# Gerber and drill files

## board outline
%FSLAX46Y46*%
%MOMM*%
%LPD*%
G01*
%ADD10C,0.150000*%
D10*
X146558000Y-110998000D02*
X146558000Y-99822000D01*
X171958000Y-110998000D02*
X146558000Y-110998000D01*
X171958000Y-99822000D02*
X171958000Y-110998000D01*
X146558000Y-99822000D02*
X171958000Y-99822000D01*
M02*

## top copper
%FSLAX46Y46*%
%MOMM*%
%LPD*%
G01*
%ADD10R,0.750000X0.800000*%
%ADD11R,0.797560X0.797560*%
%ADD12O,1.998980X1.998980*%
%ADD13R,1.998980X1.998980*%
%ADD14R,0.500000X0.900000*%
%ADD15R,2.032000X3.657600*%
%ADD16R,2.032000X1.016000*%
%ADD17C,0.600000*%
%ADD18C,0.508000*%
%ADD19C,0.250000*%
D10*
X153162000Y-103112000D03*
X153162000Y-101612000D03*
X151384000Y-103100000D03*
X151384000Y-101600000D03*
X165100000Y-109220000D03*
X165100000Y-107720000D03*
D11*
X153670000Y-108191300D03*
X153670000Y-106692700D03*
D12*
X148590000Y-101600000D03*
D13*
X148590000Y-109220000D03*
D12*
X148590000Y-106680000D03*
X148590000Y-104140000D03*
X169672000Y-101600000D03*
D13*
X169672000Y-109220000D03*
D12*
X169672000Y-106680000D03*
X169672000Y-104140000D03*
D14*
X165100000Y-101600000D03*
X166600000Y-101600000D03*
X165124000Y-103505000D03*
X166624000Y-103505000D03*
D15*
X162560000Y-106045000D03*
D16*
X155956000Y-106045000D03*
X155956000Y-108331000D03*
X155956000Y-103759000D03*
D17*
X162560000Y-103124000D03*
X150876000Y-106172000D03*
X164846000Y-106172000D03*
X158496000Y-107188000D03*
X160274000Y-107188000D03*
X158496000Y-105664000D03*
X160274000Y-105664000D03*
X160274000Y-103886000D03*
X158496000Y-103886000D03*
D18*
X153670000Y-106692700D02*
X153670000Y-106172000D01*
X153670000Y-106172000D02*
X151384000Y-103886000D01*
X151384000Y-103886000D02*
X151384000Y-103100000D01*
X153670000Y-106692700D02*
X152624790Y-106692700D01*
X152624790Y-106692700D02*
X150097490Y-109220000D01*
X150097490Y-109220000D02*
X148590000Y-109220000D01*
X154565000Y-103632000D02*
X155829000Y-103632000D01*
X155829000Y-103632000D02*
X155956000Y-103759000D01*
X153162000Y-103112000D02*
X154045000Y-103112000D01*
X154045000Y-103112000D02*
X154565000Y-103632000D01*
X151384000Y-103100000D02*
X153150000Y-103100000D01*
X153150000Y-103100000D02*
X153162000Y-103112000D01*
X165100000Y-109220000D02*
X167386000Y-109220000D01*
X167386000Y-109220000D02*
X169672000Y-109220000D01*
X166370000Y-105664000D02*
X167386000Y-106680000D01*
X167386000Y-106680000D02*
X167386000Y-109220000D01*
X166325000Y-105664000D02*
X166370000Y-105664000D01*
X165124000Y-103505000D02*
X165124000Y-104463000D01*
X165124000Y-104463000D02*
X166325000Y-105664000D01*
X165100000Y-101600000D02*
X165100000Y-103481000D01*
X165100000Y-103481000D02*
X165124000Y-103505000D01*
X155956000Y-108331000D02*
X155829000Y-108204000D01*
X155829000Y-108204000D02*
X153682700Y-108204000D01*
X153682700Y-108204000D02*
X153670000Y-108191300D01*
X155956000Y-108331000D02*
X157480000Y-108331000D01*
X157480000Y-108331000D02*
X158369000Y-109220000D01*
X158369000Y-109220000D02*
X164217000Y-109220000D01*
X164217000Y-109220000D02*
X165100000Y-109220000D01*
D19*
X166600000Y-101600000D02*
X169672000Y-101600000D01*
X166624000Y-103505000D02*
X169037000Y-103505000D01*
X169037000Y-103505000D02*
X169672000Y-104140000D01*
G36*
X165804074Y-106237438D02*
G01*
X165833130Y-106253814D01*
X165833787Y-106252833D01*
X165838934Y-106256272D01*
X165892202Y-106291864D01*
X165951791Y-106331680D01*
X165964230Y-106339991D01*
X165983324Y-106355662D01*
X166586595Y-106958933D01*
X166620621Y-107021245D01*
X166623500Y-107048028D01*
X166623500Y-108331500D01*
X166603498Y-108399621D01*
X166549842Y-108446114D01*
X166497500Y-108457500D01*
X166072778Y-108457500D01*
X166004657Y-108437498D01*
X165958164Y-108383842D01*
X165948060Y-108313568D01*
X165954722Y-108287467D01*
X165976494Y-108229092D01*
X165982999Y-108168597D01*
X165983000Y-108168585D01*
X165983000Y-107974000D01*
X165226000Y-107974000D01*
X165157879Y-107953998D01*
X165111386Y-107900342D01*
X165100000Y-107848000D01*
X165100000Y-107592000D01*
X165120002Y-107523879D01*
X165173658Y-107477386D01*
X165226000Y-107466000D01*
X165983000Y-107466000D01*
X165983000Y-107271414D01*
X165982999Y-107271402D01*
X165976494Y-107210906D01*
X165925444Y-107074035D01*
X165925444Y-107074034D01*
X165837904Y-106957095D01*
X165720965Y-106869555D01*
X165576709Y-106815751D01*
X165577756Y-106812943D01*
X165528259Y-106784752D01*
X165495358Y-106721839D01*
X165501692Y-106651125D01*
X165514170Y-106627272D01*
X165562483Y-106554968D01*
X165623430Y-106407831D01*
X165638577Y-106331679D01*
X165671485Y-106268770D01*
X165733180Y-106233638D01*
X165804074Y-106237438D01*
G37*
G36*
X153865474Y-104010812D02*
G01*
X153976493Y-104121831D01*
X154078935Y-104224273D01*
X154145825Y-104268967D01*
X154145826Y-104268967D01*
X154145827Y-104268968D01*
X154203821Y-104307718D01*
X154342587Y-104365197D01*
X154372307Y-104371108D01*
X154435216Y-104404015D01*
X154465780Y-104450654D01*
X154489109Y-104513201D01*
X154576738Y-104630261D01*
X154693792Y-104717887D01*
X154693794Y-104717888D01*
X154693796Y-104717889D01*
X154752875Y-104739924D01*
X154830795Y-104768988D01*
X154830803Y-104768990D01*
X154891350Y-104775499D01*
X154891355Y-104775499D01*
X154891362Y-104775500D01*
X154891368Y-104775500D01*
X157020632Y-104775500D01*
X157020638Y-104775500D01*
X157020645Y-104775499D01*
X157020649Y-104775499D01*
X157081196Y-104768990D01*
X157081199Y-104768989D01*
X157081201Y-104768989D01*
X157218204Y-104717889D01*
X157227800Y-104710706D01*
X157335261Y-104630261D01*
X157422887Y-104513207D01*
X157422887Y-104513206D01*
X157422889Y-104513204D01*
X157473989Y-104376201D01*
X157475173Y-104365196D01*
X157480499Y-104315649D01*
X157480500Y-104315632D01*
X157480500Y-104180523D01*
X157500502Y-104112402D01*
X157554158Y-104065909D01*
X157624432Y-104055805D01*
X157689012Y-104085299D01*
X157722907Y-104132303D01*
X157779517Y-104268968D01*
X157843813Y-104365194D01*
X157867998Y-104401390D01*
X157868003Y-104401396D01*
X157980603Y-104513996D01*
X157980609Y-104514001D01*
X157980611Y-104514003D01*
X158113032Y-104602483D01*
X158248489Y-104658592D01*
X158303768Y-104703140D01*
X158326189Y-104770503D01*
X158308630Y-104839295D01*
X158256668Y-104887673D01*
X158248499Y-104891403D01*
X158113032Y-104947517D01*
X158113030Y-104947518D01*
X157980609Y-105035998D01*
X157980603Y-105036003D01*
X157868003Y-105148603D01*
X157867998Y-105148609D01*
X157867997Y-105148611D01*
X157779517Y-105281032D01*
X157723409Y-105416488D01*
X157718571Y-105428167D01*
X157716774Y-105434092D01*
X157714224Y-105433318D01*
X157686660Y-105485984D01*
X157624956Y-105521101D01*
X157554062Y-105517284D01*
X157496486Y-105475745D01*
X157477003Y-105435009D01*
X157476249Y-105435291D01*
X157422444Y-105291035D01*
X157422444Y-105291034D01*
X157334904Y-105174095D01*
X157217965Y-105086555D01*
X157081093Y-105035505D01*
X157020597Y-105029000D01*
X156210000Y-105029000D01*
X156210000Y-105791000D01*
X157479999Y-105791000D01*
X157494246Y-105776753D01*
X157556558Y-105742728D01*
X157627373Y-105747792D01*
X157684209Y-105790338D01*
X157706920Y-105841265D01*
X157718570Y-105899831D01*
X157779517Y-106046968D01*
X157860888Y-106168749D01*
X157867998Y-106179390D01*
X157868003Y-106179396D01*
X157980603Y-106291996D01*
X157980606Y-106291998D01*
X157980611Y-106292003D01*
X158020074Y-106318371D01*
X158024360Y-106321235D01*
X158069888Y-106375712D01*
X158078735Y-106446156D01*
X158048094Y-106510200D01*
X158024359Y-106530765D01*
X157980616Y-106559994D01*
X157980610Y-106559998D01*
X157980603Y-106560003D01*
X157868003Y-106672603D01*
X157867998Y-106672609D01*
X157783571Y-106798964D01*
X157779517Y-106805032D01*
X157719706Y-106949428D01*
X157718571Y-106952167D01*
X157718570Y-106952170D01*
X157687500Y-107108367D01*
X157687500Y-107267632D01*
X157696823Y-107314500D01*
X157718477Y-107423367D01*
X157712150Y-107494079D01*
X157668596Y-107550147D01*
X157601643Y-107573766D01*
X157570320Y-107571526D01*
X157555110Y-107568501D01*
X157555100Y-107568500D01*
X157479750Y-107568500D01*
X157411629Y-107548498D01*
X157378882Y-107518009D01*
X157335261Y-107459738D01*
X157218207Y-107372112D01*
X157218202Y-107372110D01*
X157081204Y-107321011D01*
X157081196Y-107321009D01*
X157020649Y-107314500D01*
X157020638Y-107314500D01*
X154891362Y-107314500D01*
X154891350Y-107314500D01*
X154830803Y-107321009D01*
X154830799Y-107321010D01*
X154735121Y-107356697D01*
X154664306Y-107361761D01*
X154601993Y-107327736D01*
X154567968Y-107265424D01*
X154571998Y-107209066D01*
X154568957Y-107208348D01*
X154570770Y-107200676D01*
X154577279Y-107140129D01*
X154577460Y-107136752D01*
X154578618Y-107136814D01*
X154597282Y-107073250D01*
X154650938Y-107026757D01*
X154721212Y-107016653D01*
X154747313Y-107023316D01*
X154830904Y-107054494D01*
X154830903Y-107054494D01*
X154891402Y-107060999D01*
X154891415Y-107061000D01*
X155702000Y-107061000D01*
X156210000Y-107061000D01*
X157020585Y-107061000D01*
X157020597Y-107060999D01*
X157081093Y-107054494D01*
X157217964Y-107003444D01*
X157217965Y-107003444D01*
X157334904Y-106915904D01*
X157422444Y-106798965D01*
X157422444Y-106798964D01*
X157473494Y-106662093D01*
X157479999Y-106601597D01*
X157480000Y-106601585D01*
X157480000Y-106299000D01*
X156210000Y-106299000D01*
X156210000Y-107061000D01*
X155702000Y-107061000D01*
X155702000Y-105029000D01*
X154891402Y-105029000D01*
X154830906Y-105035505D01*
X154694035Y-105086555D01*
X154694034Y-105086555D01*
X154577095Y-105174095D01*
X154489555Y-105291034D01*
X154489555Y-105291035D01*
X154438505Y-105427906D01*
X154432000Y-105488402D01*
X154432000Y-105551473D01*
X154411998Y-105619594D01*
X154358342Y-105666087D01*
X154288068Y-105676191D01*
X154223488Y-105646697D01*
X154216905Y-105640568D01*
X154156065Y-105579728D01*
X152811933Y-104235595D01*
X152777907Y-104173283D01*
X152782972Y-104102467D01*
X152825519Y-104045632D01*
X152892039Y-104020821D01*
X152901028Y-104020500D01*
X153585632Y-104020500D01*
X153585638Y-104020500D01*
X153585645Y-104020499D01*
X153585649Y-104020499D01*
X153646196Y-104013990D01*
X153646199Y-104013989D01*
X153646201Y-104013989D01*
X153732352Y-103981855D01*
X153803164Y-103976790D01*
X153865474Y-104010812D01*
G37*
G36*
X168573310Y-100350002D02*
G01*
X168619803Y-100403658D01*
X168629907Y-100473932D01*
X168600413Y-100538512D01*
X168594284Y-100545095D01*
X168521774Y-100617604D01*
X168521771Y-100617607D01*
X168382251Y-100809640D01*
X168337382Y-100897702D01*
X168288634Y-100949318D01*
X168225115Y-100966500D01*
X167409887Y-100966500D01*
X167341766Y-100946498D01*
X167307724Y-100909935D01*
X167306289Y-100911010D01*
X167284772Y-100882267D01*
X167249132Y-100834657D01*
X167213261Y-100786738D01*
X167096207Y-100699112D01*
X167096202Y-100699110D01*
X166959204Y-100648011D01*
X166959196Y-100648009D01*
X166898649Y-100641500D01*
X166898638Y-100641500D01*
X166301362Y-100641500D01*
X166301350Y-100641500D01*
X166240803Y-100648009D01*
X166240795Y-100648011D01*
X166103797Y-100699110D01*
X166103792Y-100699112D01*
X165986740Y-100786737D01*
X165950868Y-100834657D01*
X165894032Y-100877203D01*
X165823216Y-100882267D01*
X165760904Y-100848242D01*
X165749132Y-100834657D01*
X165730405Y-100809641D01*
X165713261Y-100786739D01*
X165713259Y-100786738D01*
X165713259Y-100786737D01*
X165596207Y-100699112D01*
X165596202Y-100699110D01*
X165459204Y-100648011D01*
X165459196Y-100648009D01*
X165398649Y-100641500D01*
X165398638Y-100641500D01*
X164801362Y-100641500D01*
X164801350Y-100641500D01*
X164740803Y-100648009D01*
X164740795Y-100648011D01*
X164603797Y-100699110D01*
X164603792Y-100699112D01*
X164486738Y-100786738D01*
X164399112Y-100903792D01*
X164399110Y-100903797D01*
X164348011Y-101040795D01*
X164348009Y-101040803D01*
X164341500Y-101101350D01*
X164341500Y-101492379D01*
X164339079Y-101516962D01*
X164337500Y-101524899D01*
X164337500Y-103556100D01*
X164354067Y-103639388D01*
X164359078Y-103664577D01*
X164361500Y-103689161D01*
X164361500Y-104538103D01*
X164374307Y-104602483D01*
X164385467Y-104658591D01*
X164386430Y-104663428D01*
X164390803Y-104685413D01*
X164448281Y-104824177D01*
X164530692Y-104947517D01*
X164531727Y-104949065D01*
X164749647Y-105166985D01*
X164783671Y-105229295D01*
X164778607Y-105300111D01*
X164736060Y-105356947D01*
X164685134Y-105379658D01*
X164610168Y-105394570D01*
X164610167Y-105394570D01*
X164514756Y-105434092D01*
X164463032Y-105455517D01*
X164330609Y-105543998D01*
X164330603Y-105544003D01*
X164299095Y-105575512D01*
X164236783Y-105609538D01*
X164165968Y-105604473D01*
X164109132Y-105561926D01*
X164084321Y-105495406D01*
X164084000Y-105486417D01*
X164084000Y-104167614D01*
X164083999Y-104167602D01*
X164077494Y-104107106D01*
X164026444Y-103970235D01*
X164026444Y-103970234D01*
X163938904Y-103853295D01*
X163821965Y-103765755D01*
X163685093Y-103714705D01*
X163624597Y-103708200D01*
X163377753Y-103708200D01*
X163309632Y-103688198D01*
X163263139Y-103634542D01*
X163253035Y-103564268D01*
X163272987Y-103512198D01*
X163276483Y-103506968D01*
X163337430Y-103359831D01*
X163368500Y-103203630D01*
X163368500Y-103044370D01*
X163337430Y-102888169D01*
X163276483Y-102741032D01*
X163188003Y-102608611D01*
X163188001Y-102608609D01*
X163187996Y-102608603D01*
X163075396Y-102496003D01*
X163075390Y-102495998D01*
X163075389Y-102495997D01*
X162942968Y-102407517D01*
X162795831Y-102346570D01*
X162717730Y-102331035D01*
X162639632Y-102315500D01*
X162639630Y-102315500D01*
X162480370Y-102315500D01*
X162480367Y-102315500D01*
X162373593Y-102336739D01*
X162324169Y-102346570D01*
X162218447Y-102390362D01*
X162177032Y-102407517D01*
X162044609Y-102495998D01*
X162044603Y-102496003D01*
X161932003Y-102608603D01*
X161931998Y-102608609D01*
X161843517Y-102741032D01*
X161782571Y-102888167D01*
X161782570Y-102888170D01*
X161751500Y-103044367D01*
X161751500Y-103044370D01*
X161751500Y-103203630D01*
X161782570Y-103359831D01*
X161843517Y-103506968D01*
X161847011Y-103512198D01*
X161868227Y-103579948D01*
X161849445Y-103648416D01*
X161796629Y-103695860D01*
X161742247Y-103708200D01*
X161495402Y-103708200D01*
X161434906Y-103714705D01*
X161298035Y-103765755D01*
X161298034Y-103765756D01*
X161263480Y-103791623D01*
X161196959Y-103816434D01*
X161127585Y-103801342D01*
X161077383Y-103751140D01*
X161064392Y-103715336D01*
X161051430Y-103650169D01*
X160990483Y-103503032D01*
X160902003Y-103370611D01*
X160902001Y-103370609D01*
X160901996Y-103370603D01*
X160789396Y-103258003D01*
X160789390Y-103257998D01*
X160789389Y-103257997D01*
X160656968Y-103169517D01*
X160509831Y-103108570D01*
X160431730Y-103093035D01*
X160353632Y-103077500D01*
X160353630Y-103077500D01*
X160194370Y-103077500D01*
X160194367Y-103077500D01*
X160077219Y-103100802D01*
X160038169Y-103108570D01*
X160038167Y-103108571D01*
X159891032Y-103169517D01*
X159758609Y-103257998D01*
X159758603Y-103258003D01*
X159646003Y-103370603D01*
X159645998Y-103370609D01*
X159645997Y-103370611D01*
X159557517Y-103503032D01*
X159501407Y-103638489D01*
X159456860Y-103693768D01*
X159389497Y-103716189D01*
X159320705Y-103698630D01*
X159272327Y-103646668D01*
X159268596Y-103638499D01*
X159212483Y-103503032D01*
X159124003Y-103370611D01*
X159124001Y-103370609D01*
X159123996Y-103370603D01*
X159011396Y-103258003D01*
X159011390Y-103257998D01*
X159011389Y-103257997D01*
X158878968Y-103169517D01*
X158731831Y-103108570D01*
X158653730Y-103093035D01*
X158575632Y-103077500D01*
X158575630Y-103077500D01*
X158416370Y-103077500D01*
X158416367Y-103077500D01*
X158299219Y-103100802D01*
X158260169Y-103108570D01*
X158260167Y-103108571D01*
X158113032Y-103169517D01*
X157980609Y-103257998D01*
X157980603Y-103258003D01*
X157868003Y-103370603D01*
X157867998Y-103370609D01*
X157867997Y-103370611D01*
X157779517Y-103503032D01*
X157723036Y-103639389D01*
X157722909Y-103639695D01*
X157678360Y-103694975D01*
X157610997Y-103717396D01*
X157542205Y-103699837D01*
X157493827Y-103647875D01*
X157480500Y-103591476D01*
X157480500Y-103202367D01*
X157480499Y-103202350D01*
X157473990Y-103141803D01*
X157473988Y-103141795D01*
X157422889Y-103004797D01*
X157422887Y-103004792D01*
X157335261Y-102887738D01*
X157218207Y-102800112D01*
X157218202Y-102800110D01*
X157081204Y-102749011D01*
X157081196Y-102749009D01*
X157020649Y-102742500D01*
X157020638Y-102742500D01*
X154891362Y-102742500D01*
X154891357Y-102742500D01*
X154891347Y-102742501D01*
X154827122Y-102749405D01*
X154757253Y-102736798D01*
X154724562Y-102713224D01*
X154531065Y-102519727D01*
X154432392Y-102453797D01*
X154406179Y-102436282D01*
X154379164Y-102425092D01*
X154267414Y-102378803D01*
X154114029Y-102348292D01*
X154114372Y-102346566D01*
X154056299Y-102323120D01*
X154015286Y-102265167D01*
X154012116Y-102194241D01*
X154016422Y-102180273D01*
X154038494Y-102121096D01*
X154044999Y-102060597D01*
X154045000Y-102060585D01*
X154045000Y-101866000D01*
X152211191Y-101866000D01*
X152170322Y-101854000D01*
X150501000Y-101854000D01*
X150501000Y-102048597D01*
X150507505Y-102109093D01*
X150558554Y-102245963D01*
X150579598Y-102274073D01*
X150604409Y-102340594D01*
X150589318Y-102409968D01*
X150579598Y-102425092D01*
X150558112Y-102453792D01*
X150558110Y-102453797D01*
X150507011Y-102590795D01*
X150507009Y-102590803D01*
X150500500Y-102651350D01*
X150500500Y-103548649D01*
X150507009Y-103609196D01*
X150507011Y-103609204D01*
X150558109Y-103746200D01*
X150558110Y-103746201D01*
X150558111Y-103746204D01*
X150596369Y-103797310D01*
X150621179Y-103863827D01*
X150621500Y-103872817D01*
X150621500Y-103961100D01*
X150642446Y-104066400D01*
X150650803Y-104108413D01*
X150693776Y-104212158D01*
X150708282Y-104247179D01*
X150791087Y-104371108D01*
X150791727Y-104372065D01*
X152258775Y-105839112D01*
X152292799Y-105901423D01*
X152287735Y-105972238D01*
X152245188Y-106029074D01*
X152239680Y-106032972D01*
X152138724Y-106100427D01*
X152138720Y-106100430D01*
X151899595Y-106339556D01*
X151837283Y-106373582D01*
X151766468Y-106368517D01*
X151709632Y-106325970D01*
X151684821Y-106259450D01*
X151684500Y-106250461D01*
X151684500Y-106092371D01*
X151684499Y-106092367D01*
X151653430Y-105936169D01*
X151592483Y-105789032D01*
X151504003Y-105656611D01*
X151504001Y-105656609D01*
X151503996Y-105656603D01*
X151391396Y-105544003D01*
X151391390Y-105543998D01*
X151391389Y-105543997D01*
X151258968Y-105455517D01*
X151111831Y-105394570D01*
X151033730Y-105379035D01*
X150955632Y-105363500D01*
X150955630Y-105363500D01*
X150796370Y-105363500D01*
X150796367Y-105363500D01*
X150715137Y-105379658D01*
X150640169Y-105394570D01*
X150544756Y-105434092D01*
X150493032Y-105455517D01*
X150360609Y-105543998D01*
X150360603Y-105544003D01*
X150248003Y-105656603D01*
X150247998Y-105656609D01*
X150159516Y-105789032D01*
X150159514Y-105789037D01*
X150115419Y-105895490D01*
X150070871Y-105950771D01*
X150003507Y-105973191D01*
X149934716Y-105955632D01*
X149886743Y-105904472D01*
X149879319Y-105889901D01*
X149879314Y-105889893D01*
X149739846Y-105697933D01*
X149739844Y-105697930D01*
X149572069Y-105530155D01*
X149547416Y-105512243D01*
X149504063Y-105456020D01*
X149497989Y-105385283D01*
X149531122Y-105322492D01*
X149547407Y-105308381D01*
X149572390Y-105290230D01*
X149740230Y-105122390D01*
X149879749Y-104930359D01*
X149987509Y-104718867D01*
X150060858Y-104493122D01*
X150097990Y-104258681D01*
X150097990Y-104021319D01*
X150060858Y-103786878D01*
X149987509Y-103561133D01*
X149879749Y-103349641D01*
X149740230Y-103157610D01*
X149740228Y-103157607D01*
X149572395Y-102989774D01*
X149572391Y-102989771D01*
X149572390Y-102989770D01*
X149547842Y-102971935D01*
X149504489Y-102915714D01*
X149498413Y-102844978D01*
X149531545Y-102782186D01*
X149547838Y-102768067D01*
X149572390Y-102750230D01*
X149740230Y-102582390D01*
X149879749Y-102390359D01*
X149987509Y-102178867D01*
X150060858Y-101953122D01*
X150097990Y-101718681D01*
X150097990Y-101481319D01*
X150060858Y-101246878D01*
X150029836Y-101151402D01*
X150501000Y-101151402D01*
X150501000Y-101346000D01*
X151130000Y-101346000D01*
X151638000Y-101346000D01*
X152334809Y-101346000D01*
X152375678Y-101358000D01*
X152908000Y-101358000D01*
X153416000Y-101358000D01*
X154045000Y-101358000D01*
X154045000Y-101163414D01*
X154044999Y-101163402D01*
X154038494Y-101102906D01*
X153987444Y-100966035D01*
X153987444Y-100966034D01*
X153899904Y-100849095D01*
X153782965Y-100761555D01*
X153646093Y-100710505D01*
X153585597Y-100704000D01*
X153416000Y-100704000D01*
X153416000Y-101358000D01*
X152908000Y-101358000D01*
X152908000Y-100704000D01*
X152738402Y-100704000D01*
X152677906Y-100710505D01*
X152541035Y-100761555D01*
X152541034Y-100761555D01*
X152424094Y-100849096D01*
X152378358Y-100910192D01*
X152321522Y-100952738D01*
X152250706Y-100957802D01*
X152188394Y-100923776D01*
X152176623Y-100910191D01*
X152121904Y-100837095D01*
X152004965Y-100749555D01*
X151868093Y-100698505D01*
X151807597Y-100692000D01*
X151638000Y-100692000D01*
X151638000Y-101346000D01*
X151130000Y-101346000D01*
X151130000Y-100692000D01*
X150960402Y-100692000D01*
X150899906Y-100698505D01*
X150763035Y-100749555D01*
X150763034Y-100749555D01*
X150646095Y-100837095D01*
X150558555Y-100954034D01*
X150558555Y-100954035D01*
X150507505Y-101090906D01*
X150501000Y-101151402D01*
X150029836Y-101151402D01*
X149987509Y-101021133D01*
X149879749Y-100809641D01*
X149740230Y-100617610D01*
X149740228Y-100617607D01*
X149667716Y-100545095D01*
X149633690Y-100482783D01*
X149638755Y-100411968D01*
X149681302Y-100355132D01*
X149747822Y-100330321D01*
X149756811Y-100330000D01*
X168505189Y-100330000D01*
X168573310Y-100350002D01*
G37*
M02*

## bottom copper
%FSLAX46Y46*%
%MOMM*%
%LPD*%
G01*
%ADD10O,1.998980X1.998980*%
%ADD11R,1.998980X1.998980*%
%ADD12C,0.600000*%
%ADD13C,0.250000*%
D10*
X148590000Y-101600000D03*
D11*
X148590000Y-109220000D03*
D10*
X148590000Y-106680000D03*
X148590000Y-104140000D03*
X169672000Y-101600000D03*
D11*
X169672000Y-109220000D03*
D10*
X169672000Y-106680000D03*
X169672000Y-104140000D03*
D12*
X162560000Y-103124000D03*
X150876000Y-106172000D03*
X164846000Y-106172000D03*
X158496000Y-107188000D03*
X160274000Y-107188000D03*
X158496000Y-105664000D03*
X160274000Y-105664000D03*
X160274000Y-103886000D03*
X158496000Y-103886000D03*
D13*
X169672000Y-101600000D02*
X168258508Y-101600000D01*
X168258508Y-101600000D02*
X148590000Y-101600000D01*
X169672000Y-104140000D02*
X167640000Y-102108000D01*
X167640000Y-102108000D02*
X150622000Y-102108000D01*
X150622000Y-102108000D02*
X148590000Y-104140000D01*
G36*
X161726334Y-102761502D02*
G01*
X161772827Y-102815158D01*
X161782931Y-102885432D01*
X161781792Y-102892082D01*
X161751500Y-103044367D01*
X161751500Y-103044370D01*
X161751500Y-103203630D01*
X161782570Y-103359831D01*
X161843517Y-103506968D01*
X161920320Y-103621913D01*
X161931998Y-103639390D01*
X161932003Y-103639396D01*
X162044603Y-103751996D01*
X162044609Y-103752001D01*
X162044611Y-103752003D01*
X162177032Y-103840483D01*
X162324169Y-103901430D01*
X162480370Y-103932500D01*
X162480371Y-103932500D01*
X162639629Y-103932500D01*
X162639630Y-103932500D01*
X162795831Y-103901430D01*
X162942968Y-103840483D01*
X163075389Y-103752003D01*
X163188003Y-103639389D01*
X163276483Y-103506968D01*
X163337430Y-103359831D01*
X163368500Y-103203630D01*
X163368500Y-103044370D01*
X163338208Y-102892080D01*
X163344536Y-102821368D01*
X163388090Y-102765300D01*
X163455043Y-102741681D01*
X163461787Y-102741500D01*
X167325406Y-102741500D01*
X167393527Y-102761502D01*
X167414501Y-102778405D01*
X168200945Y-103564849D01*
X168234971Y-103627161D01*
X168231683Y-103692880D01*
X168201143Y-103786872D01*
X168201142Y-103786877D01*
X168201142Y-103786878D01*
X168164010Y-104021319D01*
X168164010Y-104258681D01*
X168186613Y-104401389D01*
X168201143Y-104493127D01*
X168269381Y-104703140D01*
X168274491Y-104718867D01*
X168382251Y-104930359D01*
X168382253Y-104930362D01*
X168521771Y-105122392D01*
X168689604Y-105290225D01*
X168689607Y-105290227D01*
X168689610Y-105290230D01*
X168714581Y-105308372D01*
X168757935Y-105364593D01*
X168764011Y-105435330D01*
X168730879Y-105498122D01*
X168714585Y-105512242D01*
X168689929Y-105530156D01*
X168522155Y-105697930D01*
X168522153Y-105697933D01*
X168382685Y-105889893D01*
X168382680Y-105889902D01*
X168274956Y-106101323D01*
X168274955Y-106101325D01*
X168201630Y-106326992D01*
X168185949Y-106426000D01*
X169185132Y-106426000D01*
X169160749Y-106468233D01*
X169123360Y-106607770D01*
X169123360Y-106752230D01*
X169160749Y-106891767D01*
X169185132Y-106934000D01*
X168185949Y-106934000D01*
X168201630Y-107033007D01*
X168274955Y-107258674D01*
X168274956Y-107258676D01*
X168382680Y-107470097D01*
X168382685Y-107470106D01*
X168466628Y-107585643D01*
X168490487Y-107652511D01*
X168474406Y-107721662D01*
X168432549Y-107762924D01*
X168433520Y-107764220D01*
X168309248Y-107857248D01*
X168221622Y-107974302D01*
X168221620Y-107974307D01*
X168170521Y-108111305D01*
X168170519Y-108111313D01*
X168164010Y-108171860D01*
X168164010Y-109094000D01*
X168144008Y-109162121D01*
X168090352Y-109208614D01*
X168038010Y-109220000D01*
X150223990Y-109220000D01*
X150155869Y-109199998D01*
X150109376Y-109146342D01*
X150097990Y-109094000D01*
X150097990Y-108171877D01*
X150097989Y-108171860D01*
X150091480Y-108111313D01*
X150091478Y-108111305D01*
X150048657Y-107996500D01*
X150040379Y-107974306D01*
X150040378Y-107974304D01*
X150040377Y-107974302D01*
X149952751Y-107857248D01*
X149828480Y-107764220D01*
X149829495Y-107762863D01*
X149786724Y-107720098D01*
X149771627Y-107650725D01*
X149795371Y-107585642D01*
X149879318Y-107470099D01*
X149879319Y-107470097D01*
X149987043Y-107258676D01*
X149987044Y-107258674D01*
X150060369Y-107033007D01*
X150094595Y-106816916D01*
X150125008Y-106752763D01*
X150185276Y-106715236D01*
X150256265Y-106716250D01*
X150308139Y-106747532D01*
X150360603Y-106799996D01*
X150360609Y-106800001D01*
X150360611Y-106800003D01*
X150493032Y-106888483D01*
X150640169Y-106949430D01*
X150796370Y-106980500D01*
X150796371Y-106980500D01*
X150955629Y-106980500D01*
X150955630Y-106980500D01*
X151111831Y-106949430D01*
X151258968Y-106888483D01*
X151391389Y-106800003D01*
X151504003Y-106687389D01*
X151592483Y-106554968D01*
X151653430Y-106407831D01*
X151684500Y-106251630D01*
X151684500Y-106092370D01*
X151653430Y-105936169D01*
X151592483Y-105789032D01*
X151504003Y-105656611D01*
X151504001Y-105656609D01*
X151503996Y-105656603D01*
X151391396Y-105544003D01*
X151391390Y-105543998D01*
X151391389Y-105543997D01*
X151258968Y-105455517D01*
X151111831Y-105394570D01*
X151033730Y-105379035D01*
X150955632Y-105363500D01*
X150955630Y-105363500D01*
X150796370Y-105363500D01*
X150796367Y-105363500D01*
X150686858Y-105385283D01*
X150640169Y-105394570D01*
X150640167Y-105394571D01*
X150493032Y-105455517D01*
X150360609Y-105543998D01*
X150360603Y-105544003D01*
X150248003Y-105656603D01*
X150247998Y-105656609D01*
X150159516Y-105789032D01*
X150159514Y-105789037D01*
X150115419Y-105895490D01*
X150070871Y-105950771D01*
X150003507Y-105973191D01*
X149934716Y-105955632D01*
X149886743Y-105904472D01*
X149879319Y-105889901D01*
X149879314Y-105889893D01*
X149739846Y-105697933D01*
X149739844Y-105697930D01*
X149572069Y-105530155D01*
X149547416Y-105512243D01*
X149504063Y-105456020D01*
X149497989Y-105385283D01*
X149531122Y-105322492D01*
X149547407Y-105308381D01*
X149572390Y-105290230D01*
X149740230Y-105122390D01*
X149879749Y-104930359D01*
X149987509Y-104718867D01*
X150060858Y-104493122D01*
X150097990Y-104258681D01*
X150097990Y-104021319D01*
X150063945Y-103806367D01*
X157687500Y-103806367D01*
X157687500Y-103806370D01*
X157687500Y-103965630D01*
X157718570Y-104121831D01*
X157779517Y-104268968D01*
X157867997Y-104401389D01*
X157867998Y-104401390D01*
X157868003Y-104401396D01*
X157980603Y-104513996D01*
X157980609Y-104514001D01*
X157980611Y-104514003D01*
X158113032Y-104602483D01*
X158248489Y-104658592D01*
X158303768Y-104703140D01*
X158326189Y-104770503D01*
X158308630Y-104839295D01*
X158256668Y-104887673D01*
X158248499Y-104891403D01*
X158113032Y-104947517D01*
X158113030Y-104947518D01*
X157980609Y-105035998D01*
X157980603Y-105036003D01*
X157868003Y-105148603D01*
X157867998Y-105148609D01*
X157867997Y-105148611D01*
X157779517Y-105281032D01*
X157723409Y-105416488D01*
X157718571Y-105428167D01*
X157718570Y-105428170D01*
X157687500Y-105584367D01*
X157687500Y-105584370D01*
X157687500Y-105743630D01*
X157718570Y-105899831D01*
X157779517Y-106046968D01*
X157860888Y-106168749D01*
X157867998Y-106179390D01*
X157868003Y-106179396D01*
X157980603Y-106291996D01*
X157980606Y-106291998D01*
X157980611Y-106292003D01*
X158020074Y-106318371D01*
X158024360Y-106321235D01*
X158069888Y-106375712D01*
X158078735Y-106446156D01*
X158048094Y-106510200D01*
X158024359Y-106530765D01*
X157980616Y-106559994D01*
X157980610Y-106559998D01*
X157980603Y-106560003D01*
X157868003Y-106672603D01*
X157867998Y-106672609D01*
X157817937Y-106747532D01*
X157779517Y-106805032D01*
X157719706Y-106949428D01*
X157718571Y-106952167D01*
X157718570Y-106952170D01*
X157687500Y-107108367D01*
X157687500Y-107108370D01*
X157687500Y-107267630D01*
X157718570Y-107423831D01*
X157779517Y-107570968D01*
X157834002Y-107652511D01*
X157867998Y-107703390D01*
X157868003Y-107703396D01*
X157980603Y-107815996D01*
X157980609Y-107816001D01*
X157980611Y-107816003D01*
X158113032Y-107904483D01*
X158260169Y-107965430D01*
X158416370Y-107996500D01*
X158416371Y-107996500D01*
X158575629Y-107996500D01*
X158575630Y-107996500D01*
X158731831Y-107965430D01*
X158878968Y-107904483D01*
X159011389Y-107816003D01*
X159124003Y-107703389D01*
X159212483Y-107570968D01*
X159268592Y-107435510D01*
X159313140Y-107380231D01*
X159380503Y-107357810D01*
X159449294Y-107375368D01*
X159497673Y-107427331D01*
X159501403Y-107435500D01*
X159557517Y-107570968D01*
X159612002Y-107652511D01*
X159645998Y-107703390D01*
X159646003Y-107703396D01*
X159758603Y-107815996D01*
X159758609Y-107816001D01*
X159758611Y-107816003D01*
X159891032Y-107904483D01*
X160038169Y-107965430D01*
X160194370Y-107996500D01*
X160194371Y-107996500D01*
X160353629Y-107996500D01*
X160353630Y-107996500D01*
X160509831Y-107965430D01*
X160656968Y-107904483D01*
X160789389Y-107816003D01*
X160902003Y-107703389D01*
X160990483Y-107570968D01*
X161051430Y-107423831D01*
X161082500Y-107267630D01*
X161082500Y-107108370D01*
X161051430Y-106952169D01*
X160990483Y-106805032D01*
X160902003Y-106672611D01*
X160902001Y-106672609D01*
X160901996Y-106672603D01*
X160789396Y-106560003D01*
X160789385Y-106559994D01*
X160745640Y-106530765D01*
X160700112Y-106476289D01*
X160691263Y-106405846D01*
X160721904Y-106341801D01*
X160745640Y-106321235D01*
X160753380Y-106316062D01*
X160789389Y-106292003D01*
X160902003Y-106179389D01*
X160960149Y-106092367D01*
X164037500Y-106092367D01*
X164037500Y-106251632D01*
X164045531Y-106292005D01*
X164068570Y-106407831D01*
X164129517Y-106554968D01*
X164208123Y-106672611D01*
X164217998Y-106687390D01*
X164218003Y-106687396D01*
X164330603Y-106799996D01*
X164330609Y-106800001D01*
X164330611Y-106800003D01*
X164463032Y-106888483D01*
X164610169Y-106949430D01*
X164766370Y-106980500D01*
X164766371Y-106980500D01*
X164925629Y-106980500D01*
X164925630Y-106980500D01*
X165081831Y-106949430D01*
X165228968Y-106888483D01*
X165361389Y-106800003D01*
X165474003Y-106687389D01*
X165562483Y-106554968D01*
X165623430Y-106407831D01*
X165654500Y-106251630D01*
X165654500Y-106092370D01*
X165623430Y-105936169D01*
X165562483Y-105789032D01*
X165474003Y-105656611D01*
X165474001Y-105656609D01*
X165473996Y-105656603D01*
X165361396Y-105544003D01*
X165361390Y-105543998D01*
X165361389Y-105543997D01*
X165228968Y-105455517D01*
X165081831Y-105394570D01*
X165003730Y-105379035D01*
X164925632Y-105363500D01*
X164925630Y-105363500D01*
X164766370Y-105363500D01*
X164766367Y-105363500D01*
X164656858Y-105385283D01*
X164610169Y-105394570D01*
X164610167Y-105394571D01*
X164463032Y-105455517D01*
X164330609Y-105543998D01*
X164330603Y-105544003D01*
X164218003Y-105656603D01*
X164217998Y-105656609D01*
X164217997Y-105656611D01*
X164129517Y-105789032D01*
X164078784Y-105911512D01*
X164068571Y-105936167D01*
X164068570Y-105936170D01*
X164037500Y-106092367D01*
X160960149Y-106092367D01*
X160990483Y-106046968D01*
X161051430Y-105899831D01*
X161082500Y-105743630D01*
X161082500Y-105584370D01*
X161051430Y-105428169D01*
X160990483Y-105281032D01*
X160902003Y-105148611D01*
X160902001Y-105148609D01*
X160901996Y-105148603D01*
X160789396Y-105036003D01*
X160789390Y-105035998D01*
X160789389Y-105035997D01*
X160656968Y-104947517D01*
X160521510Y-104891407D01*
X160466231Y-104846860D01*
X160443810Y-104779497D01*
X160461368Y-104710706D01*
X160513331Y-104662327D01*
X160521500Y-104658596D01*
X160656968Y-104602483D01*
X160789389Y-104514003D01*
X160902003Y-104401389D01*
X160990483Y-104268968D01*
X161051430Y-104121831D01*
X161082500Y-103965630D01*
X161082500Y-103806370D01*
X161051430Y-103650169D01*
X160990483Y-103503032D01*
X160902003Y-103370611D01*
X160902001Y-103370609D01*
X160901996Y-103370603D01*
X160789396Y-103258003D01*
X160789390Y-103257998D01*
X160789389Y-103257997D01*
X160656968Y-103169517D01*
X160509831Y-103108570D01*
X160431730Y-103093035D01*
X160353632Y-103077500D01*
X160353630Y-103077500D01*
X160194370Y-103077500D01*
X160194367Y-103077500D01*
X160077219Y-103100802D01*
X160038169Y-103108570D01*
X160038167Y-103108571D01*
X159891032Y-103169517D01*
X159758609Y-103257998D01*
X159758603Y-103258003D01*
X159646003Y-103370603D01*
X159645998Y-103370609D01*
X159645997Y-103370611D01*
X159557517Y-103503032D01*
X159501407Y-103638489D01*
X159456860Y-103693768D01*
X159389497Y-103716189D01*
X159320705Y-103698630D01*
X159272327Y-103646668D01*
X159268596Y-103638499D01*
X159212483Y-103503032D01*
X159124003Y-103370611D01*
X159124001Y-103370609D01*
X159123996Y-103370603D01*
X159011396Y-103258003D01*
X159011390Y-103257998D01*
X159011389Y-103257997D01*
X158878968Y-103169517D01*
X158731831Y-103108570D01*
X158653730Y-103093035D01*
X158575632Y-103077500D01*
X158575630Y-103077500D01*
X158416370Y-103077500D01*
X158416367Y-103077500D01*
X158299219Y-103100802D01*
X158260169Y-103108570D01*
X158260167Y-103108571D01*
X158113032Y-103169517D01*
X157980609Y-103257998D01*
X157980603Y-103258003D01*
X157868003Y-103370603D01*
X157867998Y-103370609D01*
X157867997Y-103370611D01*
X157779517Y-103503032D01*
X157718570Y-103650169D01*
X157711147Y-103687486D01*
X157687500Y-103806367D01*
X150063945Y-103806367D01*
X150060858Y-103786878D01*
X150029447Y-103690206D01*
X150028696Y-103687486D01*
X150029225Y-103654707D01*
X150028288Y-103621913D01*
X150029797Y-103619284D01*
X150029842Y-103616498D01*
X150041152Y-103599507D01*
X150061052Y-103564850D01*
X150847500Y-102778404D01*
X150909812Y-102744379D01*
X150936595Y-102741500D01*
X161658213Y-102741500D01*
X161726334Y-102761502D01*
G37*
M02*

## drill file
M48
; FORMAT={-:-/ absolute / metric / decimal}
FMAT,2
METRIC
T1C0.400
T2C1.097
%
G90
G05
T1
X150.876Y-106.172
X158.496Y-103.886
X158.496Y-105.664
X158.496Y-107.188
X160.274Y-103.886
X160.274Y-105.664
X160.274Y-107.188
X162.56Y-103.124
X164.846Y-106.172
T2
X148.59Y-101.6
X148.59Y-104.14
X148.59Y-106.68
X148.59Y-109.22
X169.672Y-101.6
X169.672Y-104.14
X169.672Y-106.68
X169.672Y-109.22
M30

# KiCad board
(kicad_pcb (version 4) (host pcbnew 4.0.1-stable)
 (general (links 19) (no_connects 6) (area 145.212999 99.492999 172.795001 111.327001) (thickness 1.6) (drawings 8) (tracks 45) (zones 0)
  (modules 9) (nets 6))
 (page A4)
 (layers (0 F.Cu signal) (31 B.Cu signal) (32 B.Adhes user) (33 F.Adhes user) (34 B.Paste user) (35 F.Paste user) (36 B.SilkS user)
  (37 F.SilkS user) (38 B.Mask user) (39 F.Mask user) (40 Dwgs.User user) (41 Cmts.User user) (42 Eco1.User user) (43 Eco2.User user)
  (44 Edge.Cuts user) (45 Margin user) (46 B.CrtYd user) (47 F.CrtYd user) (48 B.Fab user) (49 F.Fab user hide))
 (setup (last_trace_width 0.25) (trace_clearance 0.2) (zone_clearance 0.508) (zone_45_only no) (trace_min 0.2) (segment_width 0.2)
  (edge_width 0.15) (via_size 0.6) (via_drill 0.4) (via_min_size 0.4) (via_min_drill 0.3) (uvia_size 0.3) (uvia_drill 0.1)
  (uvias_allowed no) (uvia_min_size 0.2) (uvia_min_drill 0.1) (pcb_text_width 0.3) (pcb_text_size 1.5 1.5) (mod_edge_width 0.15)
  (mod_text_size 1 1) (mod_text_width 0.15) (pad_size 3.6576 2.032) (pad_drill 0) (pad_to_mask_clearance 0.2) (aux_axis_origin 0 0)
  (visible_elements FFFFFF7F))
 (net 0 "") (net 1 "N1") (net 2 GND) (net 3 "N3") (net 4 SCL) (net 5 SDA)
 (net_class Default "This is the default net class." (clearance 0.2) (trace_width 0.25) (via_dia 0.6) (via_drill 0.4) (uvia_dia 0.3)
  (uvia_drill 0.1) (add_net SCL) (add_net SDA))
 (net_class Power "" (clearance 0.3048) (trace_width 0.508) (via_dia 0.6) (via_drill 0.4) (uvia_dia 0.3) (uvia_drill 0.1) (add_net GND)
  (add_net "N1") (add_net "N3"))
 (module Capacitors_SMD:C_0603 (layer F.Cu) (at 153.162 102.362 90)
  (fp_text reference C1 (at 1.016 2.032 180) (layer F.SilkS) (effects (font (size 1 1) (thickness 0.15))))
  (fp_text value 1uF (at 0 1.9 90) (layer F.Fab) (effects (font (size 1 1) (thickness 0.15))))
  (pad 1 smd rect (at -0.75 0 90) (size 0.8 0.75) (layers F.Cu F.Paste F.Mask) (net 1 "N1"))
  (pad 2 smd rect (at 0.75 0 90) (size 0.8 0.75) (layers F.Cu F.Paste F.Mask) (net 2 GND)))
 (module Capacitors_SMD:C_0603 (layer F.Cu) (at 151.384 102.35 90)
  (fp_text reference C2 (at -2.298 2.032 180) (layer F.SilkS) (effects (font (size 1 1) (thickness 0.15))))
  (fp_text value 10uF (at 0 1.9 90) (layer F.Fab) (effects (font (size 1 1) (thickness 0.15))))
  (pad 1 smd rect (at -0.75 0 90) (size 0.8 0.75) (layers F.Cu F.Paste F.Mask) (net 1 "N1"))
  (pad 2 smd rect (at 0.75 0 90) (size 0.8 0.75) (layers F.Cu F.Paste F.Mask) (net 2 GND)))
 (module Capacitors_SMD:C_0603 (layer F.Cu) (at 165.1 108.47 90)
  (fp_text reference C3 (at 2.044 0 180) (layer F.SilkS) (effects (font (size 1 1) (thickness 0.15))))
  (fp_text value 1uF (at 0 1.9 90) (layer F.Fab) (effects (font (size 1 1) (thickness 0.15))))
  (pad 1 smd rect (at -0.75 0 90) (size 0.8 0.75) (layers F.Cu F.Paste F.Mask) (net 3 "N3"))
  (pad 2 smd rect (at 0.75 0 90) (size 0.8 0.75) (layers F.Cu F.Paste F.Mask) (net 2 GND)))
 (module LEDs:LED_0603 (layer F.Cu) (at 153.67 107.442 270)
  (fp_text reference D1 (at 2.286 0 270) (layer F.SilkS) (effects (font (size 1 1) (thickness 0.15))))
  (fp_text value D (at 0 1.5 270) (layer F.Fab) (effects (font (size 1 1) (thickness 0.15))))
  (pad 2 smd rect (at 0.7493 0 90) (size 0.79756 0.79756) (layers F.Cu F.Paste F.Mask) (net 3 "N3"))
  (pad 1 smd rect (at -0.7493 0 90) (size 0.79756 0.79756) (layers F.Cu F.Paste F.Mask) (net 1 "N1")))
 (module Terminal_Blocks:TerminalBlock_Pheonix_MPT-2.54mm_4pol (layer F.Cu) (at 148.59 109.22 90)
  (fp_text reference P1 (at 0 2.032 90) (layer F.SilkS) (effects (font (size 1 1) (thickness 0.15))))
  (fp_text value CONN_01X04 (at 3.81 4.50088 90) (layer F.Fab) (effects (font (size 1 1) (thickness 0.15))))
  (pad 4 thru_hole oval (at 7.62 0 270) (size 1.99898 1.99898) (drill 1.09728) (layers *.Cu *.Mask F.SilkS) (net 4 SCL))
  (pad 1 thru_hole rect (at 0 0 270) (size 1.99898 1.99898) (drill 1.09728) (layers *.Cu *.Mask F.SilkS) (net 1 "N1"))
  (pad 2 thru_hole oval (at 2.54 0 270) (size 1.99898 1.99898) (drill 1.09728) (layers *.Cu *.Mask F.SilkS) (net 2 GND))
  (pad 3 thru_hole oval (at 5.08 0 270) (size 1.99898 1.99898) (drill 1.09728) (layers *.Cu *.Mask F.SilkS) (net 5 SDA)))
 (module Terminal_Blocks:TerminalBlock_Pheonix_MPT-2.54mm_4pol (layer F.Cu) (at 169.672 109.22 90)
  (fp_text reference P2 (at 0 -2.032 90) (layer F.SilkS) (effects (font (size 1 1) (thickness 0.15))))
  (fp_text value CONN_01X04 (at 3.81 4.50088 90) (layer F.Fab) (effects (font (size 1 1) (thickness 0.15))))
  (pad 4 thru_hole oval (at 7.62 0 270) (size 1.99898 1.99898) (drill 1.09728) (layers *.Cu *.Mask F.SilkS) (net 4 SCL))
  (pad 1 thru_hole rect (at 0 0 270) (size 1.99898 1.99898) (drill 1.09728) (layers *.Cu *.Mask F.SilkS) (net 3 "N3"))
  (pad 2 thru_hole oval (at 2.54 0 270) (size 1.99898 1.99898) (drill 1.09728) (layers *.Cu *.Mask F.SilkS) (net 2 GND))
  (pad 3 thru_hole oval (at 5.08 0 270) (size 1.99898 1.99898) (drill 1.09728) (layers *.Cu *.Mask F.SilkS) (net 5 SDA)))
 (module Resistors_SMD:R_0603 (layer F.Cu) (at 165.85 101.6)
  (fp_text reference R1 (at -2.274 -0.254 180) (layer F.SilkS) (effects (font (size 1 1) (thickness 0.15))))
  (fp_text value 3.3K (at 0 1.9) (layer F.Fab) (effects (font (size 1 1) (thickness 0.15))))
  (pad 1 smd rect (at -0.75 0) (size 0.5 0.9) (layers F.Cu F.Paste F.Mask) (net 3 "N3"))
  (pad 2 smd rect (at 0.75 0) (size 0.5 0.9) (layers F.Cu F.Paste F.Mask) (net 4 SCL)))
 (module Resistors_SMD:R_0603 (layer F.Cu) (at 165.874 103.505)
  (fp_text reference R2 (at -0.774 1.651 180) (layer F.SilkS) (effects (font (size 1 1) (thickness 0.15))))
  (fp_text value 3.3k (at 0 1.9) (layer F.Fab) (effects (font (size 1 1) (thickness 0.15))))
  (pad 1 smd rect (at -0.75 0) (size 0.5 0.9) (layers F.Cu F.Paste F.Mask) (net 3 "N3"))
  (pad 2 smd rect (at 0.75 0) (size 0.5 0.9) (layers F.Cu F.Paste F.Mask) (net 5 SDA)))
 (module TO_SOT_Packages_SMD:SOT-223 (layer F.Cu) (at 159.258 106.045 270)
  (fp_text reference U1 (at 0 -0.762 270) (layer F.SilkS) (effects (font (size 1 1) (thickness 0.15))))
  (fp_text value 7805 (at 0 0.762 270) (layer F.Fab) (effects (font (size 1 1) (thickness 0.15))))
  (pad GND smd rect (at 0 -3.302 270) (size 3.6576 2.032) (layers F.Cu F.Paste F.Mask) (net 2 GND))
  (pad GND smd rect (at 0 3.302 270) (size 1.016 2.032) (layers F.Cu F.Paste F.Mask) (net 2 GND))
  (pad VO smd rect (at 2.286 3.302 270) (size 1.016 2.032) (layers F.Cu F.Paste F.Mask) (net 3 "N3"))
  (pad VI smd rect (at -2.286 3.302 270) (size 1.016 2.032) (layers F.Cu F.Paste F.Mask) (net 1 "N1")))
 (gr_line (start 146.558 110.998) (end 146.558 99.822) (layer Edge.Cuts) (width 0.15))
 (gr_line (start 171.958 110.998) (end 146.558 110.998) (layer Edge.Cuts) (width 0.15))
 (gr_line (start 171.958 99.822) (end 171.958 110.998) (layer Edge.Cuts) (width 0.15))
 (gr_line (start 146.558 99.822) (end 171.958 99.822) (layer Edge.Cuts) (width 0.15))
 (via (at 162.56 103.124) (size 0.6) (drill 0.4) (layers F.Cu B.Cu) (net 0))
 (via (at 150.876 106.172) (size 0.6) (drill 0.4) (layers F.Cu B.Cu) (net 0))
 (via (at 164.846 106.172) (size 0.6) (drill 0.4) (layers F.Cu B.Cu) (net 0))
 (via (at 158.496 107.188) (size 0.6) (drill 0.4) (layers F.Cu B.Cu) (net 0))
 (via (at 160.274 107.188) (size 0.6) (drill 0.4) (layers F.Cu B.Cu) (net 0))
 (via (at 158.496 105.664) (size 0.6) (drill 0.4) (layers F.Cu B.Cu) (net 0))
 (via (at 160.274 105.664) (size 0.6) (drill 0.4) (layers F.Cu B.Cu) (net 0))
 (via (at 160.274 103.886) (size 0.6) (drill 0.4) (layers F.Cu B.Cu) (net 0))
 (via (at 158.496 103.886) (size 0.6) (drill 0.4) (layers F.Cu B.Cu) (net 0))
 (segment (start 153.67 106.6927) (end 153.67 106.172) (width 0.508) (layer F.Cu) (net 1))
 (segment (start 153.67 106.172) (end 151.384 103.886) (width 0.508) (layer F.Cu) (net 1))
 (segment (start 151.384 103.886) (end 151.384 103.1) (width 0.508) (layer F.Cu) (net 1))
 (segment (start 153.67 106.6927) (end 152.62479 106.6927) (width 0.508) (layer F.Cu) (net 1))
 (segment (start 152.62479 106.6927) (end 150.09749 109.22) (width 0.508) (layer F.Cu) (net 1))
 (segment (start 150.09749 109.22) (end 148.59 109.22) (width 0.508) (layer F.Cu) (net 1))
 (segment (start 154.565 103.632) (end 155.829 103.632) (width 0.508) (layer F.Cu) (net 1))
 (segment (start 155.829 103.632) (end 155.956 103.759) (width 0.508) (layer F.Cu) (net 1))
 (segment (start 153.162 103.112) (end 154.045 103.112) (width 0.508) (layer F.Cu) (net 1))
 (segment (start 154.045 103.112) (end 154.565 103.632) (width 0.508) (layer F.Cu) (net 1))
 (segment (start 151.384 103.1) (end 153.15 103.1) (width 0.508) (layer F.Cu) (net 1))
 (segment (start 153.15 103.1) (end 153.162 103.112) (width 0.508) (layer F.Cu) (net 1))
 (segment (start 165.1 109.22) (end 167.386 109.22) (width 0.508) (layer F.Cu) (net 3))
 (segment (start 167.386 109.22) (end 169.672 109.22) (width 0.508) (layer F.Cu) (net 3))
 (segment (start 166.37 105.664) (end 167.386 106.68) (width 0.508) (layer F.Cu) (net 3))
 (segment (start 167.386 106.68) (end 167.386 109.22) (width 0.508) (layer F.Cu) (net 3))
 (segment (start 166.325 105.664) (end 166.37 105.664) (width 0.508) (layer F.Cu) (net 3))
 (segment (start 165.124 103.505) (end 165.124 104.463) (width 0.508) (layer F.Cu) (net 3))
 (segment (start 165.124 104.463) (end 166.325 105.664) (width 0.508) (layer F.Cu) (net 3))
 (segment (start 165.1 101.6) (end 165.1 103.481) (width 0.508) (layer F.Cu) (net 3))
 (segment (start 165.1 103.481) (end 165.124 103.505) (width 0.508) (layer F.Cu) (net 3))
 (segment (start 155.956 108.331) (end 155.829 108.204) (width 0.508) (layer F.Cu) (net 3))
 (segment (start 155.829 108.204) (end 153.6827 108.204) (width 0.508) (layer F.Cu) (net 3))
 (segment (start 153.6827 108.204) (end 153.67 108.1913) (width 0.508) (layer F.Cu) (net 3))
 (segment (start 155.956 108.331) (end 157.48 108.331) (width 0.508) (layer F.Cu) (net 3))
 (segment (start 157.48 108.331) (end 158.369 109.22) (width 0.508) (layer F.Cu) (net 3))
 (segment (start 158.369 109.22) (end 164.217 109.22) (width 0.508) (layer F.Cu) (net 3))
 (segment (start 164.217 109.22) (end 165.1 109.22) (width 0.508) (layer F.Cu) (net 3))
 (segment (start 166.6 101.6) (end 169.672 101.6) (width 0.25) (layer F.Cu) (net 4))
 (segment (start 169.672 101.6) (end 168.258508 101.6) (width 0.25) (layer B.Cu) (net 4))
 (segment (start 168.258508 101.6) (end 148.59 101.6) (width 0.25) (layer B.Cu) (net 4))
 (segment (start 166.624 103.505) (end 169.037 103.505) (width 0.25) (layer F.Cu) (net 5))
 (segment (start 169.037 103.505) (end 169.672 104.14) (width 0.25) (layer F.Cu) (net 5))
 (segment (start 169.672 104.14) (end 167.64 102.108) (width 0.25) (layer B.Cu) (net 5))
 (segment (start 167.64 102.108) (end 150.622 102.108) (width 0.25) (layer B.Cu) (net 5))
 (segment (start 150.622 102.108) (end 148.59 104.14) (width 0.25) (layer B.Cu) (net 5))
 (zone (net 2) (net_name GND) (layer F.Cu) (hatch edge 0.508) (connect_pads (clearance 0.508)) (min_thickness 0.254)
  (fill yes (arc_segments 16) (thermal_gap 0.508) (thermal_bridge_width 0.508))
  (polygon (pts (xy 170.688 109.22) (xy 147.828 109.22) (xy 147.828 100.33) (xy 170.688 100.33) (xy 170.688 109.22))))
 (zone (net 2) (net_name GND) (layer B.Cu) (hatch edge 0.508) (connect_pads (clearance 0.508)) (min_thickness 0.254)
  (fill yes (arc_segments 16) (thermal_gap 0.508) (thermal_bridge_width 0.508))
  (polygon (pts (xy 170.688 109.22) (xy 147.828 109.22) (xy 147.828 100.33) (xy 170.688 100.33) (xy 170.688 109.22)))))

